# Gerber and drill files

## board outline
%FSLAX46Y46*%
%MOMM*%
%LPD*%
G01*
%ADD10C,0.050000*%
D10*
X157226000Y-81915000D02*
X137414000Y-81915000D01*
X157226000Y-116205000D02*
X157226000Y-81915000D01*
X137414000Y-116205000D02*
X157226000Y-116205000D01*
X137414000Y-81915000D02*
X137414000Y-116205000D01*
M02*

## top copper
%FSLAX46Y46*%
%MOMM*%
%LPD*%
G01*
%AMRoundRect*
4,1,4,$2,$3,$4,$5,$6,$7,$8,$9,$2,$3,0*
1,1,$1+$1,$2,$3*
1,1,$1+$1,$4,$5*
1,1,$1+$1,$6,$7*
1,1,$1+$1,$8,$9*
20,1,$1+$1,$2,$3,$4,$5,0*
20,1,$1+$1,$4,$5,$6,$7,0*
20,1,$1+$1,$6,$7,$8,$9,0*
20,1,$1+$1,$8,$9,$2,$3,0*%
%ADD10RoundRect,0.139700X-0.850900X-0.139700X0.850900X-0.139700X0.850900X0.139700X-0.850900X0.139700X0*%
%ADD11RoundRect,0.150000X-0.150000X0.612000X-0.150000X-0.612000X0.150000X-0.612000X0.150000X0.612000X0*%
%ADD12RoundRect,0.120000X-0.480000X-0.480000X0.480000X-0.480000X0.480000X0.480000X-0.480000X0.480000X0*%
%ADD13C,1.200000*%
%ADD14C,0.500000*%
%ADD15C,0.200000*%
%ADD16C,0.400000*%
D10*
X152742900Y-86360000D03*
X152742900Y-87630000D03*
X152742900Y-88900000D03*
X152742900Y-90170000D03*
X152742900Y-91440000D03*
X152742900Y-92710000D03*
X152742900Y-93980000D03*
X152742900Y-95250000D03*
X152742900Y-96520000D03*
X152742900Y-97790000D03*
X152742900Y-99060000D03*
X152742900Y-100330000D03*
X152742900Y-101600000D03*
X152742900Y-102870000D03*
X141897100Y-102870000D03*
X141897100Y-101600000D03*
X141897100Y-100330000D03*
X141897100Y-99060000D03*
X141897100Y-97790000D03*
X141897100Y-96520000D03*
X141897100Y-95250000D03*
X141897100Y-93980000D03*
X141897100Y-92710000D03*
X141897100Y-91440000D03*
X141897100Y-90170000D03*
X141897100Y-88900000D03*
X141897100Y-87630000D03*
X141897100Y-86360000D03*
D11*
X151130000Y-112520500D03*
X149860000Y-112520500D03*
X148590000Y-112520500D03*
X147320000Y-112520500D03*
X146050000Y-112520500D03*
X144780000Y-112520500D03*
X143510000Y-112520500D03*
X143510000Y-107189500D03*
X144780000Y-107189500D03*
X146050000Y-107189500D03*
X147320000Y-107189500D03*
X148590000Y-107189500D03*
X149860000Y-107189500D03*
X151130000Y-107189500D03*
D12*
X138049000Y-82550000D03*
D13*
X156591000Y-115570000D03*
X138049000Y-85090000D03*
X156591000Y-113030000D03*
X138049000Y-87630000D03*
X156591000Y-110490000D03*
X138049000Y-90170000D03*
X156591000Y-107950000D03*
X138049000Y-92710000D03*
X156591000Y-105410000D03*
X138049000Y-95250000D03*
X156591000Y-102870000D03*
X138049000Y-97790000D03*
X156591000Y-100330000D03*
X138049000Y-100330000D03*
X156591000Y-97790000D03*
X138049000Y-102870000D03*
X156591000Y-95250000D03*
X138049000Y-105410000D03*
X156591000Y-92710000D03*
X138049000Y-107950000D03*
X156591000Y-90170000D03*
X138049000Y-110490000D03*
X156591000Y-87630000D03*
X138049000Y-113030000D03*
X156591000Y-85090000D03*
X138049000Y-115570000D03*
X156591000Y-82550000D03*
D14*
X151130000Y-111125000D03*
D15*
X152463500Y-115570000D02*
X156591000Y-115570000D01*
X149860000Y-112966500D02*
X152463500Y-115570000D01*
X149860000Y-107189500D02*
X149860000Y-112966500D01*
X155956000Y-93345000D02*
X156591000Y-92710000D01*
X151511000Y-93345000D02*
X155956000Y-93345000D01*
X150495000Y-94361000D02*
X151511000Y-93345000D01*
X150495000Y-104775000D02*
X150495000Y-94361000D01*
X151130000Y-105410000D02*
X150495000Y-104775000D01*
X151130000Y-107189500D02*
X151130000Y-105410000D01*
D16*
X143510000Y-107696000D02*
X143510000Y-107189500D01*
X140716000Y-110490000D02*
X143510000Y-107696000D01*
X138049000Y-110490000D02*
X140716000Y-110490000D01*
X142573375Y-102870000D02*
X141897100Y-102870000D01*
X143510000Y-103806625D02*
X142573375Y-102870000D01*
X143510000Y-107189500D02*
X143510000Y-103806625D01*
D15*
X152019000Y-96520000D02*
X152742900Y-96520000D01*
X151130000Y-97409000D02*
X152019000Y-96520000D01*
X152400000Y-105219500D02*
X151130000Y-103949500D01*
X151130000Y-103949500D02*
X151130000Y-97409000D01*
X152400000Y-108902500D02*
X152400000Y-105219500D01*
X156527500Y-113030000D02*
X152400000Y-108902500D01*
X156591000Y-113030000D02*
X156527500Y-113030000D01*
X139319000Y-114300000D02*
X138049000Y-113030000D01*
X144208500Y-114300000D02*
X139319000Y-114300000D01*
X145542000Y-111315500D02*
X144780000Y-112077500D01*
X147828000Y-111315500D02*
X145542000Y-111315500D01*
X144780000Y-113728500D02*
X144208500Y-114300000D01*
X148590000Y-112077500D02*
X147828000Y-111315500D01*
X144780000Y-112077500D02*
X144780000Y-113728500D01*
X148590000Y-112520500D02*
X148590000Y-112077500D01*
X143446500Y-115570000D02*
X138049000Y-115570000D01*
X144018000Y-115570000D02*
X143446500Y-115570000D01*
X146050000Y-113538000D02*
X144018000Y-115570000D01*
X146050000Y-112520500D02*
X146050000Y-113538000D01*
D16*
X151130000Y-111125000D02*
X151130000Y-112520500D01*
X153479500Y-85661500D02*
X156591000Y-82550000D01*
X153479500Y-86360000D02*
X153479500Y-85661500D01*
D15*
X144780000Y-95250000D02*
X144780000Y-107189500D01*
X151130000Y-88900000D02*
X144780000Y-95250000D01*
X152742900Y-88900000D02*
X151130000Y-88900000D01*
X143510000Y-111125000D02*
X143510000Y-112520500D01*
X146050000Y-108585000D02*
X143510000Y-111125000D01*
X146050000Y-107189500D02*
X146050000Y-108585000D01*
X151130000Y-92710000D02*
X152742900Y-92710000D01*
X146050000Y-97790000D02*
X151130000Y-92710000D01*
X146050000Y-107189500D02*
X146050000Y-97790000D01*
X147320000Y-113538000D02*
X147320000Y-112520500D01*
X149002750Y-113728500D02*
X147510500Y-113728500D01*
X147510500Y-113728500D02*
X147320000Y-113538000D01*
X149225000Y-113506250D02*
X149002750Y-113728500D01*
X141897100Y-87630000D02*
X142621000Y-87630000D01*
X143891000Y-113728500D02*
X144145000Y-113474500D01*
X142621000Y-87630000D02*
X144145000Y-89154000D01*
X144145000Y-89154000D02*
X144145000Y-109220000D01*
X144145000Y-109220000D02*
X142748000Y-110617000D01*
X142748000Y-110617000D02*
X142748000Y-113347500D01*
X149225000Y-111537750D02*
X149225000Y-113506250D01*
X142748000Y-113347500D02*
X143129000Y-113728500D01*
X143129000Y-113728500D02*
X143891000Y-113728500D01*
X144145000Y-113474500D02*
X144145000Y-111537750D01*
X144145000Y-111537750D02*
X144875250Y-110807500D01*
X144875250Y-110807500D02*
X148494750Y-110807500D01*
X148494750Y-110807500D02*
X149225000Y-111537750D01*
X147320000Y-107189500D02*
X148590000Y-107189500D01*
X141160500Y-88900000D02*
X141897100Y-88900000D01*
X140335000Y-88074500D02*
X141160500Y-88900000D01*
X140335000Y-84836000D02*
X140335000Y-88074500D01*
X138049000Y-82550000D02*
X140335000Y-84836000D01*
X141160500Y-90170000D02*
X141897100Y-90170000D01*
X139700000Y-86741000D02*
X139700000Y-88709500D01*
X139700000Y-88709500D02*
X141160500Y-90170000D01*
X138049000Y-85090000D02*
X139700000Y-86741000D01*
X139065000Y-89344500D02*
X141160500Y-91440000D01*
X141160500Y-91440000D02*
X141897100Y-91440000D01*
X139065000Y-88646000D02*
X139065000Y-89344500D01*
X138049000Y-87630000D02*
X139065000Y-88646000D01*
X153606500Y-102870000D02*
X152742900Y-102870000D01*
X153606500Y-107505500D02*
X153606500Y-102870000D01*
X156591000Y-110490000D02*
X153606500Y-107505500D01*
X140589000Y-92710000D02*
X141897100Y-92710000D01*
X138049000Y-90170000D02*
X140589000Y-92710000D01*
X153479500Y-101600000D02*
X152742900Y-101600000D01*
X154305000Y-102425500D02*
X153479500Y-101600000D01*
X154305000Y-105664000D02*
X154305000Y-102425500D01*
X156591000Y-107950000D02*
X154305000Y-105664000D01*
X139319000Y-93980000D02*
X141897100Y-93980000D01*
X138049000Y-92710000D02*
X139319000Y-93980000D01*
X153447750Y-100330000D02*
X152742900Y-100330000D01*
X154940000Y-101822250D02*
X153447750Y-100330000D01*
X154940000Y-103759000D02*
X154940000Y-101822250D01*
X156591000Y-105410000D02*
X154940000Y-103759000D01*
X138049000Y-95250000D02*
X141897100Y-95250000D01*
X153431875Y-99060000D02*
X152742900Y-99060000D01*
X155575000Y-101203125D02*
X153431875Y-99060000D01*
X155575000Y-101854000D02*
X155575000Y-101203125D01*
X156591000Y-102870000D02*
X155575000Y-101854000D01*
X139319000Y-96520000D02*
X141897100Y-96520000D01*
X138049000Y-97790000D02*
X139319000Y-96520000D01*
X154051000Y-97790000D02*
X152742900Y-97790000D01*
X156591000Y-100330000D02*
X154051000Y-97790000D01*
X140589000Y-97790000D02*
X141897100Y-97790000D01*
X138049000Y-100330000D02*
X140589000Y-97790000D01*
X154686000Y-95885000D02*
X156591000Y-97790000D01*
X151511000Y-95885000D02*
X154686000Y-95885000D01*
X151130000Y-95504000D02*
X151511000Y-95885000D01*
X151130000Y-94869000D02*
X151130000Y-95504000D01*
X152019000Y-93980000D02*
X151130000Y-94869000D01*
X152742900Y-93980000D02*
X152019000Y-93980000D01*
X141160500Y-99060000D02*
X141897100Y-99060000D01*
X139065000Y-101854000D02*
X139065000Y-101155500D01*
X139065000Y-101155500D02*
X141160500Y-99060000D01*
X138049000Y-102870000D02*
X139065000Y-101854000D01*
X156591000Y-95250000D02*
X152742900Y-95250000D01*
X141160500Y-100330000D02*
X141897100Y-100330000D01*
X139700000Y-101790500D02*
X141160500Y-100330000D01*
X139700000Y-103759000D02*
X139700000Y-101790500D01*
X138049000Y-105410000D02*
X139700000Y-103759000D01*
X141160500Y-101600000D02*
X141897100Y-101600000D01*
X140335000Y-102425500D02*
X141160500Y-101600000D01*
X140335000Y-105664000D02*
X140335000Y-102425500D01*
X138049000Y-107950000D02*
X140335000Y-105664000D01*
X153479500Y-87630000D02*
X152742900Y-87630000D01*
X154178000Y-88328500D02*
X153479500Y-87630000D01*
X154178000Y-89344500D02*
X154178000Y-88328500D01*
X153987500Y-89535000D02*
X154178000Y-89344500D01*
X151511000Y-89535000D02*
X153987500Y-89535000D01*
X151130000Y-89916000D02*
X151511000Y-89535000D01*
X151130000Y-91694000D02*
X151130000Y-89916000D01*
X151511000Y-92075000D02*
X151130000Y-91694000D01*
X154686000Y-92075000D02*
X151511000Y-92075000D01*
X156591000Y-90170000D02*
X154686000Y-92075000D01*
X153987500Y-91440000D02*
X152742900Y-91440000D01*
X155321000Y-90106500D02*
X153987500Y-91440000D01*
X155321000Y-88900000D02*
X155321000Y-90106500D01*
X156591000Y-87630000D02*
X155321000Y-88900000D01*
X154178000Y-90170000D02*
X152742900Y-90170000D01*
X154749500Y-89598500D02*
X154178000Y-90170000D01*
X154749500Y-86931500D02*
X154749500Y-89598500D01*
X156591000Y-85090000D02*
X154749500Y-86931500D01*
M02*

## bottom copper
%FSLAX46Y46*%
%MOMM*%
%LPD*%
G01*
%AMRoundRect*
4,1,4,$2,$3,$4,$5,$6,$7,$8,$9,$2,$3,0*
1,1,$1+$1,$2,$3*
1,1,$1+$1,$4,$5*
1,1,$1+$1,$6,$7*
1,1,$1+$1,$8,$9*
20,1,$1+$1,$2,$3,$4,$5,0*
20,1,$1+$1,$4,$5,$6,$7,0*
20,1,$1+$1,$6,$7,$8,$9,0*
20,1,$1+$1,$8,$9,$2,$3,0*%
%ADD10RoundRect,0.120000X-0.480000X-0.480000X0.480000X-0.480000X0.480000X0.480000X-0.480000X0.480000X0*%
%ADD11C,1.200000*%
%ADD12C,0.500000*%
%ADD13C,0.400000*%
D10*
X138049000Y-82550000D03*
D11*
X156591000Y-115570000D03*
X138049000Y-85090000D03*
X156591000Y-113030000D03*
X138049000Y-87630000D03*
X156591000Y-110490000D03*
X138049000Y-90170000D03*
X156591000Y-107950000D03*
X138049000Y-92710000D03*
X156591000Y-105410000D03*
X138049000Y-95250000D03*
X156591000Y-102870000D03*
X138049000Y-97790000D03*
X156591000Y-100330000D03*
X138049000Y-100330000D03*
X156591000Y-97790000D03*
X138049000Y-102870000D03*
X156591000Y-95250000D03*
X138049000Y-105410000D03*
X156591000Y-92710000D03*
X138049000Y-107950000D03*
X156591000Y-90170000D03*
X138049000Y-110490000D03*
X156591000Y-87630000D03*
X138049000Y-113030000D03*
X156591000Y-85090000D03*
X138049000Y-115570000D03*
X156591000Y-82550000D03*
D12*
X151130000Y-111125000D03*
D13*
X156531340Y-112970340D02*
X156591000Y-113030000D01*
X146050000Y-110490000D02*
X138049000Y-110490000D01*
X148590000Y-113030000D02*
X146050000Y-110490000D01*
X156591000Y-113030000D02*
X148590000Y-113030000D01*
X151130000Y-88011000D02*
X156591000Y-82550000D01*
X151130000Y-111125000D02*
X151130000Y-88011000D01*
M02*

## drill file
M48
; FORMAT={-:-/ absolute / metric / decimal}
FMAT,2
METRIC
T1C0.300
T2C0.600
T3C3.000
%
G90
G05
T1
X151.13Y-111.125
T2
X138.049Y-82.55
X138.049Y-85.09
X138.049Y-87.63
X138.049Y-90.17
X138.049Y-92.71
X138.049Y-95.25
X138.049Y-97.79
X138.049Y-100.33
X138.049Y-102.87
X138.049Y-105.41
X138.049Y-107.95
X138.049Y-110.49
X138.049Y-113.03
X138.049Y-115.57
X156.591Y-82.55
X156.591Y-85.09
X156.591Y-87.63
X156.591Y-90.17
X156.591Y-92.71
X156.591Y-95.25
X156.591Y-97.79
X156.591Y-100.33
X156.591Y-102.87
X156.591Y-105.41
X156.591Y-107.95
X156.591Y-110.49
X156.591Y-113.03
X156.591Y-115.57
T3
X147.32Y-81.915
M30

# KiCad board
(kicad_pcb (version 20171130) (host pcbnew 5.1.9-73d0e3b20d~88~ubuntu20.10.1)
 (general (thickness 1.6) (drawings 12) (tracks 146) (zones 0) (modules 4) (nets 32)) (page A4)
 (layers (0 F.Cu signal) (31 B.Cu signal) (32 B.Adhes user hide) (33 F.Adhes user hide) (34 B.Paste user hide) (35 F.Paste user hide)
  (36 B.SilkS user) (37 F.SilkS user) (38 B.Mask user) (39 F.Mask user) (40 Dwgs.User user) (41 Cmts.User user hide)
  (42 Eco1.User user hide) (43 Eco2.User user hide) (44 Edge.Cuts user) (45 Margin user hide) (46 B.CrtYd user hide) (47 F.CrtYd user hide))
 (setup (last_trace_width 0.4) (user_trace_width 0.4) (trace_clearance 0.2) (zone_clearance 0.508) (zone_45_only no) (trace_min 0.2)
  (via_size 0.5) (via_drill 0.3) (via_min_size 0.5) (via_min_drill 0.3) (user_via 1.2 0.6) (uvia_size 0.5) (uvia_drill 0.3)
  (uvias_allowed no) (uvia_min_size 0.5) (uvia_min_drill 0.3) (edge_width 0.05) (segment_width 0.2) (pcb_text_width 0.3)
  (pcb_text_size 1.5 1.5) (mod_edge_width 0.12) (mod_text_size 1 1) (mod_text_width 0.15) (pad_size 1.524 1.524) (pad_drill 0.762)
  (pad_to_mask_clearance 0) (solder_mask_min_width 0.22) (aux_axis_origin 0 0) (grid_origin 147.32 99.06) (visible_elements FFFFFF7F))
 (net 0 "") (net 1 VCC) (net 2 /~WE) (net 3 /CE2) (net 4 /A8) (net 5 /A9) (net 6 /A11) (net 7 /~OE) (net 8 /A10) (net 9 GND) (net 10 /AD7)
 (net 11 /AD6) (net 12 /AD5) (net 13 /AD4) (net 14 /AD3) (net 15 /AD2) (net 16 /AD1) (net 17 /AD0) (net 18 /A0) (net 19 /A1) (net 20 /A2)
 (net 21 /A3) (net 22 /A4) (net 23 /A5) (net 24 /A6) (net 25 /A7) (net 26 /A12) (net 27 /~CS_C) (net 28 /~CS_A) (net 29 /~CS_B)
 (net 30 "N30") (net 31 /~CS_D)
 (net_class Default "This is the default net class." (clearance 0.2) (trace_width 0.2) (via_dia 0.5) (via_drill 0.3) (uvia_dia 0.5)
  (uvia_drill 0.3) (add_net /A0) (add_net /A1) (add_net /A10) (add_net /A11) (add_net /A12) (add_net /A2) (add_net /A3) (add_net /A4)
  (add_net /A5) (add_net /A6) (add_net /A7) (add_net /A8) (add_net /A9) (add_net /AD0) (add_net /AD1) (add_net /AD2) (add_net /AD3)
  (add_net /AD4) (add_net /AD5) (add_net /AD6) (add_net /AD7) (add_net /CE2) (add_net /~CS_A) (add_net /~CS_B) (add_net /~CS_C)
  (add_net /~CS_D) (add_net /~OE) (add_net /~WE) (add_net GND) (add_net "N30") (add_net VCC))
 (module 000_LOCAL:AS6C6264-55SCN (layer F.Cu) (at 147.32 94.615)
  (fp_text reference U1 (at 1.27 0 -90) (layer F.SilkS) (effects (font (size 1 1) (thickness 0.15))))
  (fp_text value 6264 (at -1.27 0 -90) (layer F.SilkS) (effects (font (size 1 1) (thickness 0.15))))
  (pad 28 smd roundrect (at 5.4229 -8.255) (size 1.9812 0.5588) (layers F.Cu F.Paste F.Mask) (roundrect_rratio 0.25) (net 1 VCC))
  (pad 27 smd roundrect (at 5.4229 -6.985) (size 1.9812 0.5588) (layers F.Cu F.Paste F.Mask) (roundrect_rratio 0.25) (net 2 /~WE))
  (pad 26 smd roundrect (at 5.4229 -5.715) (size 1.9812 0.5588) (layers F.Cu F.Paste F.Mask) (roundrect_rratio 0.25) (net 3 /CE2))
  (pad 25 smd roundrect (at 5.4229 -4.445) (size 1.9812 0.5588) (layers F.Cu F.Paste F.Mask) (roundrect_rratio 0.25) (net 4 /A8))
  (pad 24 smd roundrect (at 5.4229 -3.175) (size 1.9812 0.5588) (layers F.Cu F.Paste F.Mask) (roundrect_rratio 0.25) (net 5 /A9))
  (pad 23 smd roundrect (at 5.4229 -1.905) (size 1.9812 0.5588) (layers F.Cu F.Paste F.Mask) (roundrect_rratio 0.25) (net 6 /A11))
  (pad 22 smd roundrect (at 5.4229 -0.635) (size 1.9812 0.5588) (layers F.Cu F.Paste F.Mask) (roundrect_rratio 0.25) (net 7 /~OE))
  (pad 21 smd roundrect (at 5.4229 0.635) (size 1.9812 0.5588) (layers F.Cu F.Paste F.Mask) (roundrect_rratio 0.25) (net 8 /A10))
  (pad 20 smd roundrect (at 5.4229 1.905) (size 1.9812 0.5588) (layers F.Cu F.Paste F.Mask) (roundrect_rratio 0.25) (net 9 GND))
  (pad 19 smd roundrect (at 5.4229 3.175) (size 1.9812 0.5588) (layers F.Cu F.Paste F.Mask) (roundrect_rratio 0.25) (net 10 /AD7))
  (pad 18 smd roundrect (at 5.4229 4.445) (size 1.9812 0.5588) (layers F.Cu F.Paste F.Mask) (roundrect_rratio 0.25) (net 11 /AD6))
  (pad 17 smd roundrect (at 5.4229 5.715) (size 1.9812 0.5588) (layers F.Cu F.Paste F.Mask) (roundrect_rratio 0.25) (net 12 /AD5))
  (pad 16 smd roundrect (at 5.4229 6.985) (size 1.9812 0.5588) (layers F.Cu F.Paste F.Mask) (roundrect_rratio 0.25) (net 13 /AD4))
  (pad 15 smd roundrect (at 5.4229 8.255) (size 1.9812 0.5588) (layers F.Cu F.Paste F.Mask) (roundrect_rratio 0.25) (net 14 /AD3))
  (pad 14 smd roundrect (at -5.4229 8.255) (size 1.9812 0.5588) (layers F.Cu F.Paste F.Mask) (roundrect_rratio 0.25) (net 9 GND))
  (pad 13 smd roundrect (at -5.4229 6.985) (size 1.9812 0.5588) (layers F.Cu F.Paste F.Mask) (roundrect_rratio 0.25) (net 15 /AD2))
  (pad 12 smd roundrect (at -5.4229 5.715) (size 1.9812 0.5588) (layers F.Cu F.Paste F.Mask) (roundrect_rratio 0.25) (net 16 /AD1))
  (pad 11 smd roundrect (at -5.4229 4.445) (size 1.9812 0.5588) (layers F.Cu F.Paste F.Mask) (roundrect_rratio 0.25) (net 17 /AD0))
  (pad 10 smd roundrect (at -5.4229 3.175) (size 1.9812 0.5588) (layers F.Cu F.Paste F.Mask) (roundrect_rratio 0.25) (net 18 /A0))
  (pad 9 smd roundrect (at -5.4229 1.905) (size 1.9812 0.5588) (layers F.Cu F.Paste F.Mask) (roundrect_rratio 0.25) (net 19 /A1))
  (pad 8 smd roundrect (at -5.4229 0.635) (size 1.9812 0.5588) (layers F.Cu F.Paste F.Mask) (roundrect_rratio 0.25) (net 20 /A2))
  (pad 7 smd roundrect (at -5.4229 -0.635) (size 1.9812 0.5588) (layers F.Cu F.Paste F.Mask) (roundrect_rratio 0.25) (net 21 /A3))
  (pad 6 smd roundrect (at -5.4229 -1.905) (size 1.9812 0.5588) (layers F.Cu F.Paste F.Mask) (roundrect_rratio 0.25) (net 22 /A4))
  (pad 5 smd roundrect (at -5.4229 -3.175) (size 1.9812 0.5588) (layers F.Cu F.Paste F.Mask) (roundrect_rratio 0.25) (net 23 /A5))
  (pad 4 smd roundrect (at -5.4229 -4.445) (size 1.9812 0.5588) (layers F.Cu F.Paste F.Mask) (roundrect_rratio 0.25) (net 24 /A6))
  (pad 3 smd roundrect (at -5.4229 -5.715) (size 1.9812 0.5588) (layers F.Cu F.Paste F.Mask) (roundrect_rratio 0.25) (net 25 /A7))
  (pad 2 smd roundrect (at -5.4229 -6.985) (size 1.9812 0.5588) (layers F.Cu F.Paste F.Mask) (roundrect_rratio 0.25) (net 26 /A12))
  (pad 1 smd roundrect (at -5.4229 -8.255) (size 1.9812 0.5588) (layers F.Cu F.Paste F.Mask) (roundrect_rratio 0.25)))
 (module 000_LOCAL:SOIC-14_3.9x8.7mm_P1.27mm (layer F.Cu) (at 147.32 109.855 270) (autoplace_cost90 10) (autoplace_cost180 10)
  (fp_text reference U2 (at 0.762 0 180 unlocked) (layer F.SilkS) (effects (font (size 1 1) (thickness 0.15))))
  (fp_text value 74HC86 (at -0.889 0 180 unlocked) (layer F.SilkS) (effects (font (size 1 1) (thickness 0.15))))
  (pad 14 smd roundrect (at 2.6655 -3.81 270) (size 1.524 0.6) (layers F.Cu F.Paste F.Mask) (roundrect_rratio 0.25) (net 1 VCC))
  (pad 13 smd roundrect (at 2.6655 -2.54 270) (size 1.524 0.6) (layers F.Cu F.Paste F.Mask) (roundrect_rratio 0.25) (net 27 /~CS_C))
  (pad 12 smd roundrect (at 2.6655 -1.27 270) (size 1.524 0.6) (layers F.Cu F.Paste F.Mask) (roundrect_rratio 0.25) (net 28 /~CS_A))
  (pad 11 smd roundrect (at 2.6655 0 270) (size 1.524 0.6) (layers F.Cu F.Paste F.Mask) (roundrect_rratio 0.25) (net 26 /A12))
  (pad 10 smd roundrect (at 2.6655 1.27 270) (size 1.524 0.6) (layers F.Cu F.Paste F.Mask) (roundrect_rratio 0.25) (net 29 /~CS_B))
  (pad 9 smd roundrect (at 2.6655 2.54 270) (size 1.524 0.6) (layers F.Cu F.Paste F.Mask) (roundrect_rratio 0.25) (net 28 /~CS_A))
  (pad 8 smd roundrect (at 2.6655 3.81 270) (size 1.524 0.6) (layers F.Cu F.Paste F.Mask) (roundrect_rratio 0.25) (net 6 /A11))
  (pad 7 smd roundrect (at -2.6655 3.81 270) (size 1.524 0.6) (layers F.Cu F.Paste F.Mask) (roundrect_rratio 0.25) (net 9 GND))
  (pad 6 smd roundrect (at -2.6655 2.54 270) (size 1.524 0.6) (layers F.Cu F.Paste F.Mask) (roundrect_rratio 0.25) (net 3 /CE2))
  (pad 5 smd roundrect (at -2.6655 1.27 270) (size 1.524 0.6) (layers F.Cu F.Paste F.Mask) (roundrect_rratio 0.25) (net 6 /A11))
  (pad 4 smd roundrect (at -2.6655 0 270) (size 1.524 0.6) (layers F.Cu F.Paste F.Mask) (roundrect_rratio 0.25) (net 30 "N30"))
  (pad 3 smd roundrect (at -2.6655 -1.27 270) (size 1.524 0.6) (layers F.Cu F.Paste F.Mask) (roundrect_rratio 0.25) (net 30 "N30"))
  (pad 2 smd roundrect (at -2.6655 -2.54 270) (size 1.524 0.6) (layers F.Cu F.Paste F.Mask) (roundrect_rratio 0.25) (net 27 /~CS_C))
  (pad 1 smd roundrect (at -2.6655 -3.81 270) (size 1.524 0.6) (layers F.Cu F.Paste F.Mask) (roundrect_rratio 0.25) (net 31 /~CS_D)))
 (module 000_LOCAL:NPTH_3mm (layer F.Cu) (at 147.32 81.915)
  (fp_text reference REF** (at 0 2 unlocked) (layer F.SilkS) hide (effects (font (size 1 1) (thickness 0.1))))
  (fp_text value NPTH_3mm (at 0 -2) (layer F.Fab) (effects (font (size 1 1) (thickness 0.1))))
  (pad "" np_thru_hole circle (at 0 0) (size 3 3) (drill 3) (layers *.Cu *.Mask)))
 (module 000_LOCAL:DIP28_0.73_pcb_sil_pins (layer F.Cu) (at 147.32 99.06)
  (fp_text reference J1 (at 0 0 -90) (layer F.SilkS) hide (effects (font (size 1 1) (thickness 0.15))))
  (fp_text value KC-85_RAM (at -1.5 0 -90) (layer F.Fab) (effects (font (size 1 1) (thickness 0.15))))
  (pad 1 thru_hole roundrect (at -9.271 -16.51) (size 1.2 1.2) (drill 0.6) (layers *.Cu *.Mask) (roundrect_rratio 0.1) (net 25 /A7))
  (pad 15 thru_hole circle (at 9.271 16.51) (size 1.2 1.2) (drill 0.6) (layers *.Cu *.Mask) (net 27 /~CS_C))
  (pad 2 thru_hole circle (at -9.271 -13.97) (size 1.2 1.2) (drill 0.6) (layers *.Cu *.Mask) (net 24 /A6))
  (pad 16 thru_hole circle (at 9.271 13.97) (size 1.2 1.2) (drill 0.6) (layers *.Cu *.Mask) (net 9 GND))
  (pad 3 thru_hole circle (at -9.271 -11.43) (size 1.2 1.2) (drill 0.6) (layers *.Cu *.Mask) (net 23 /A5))
  (pad 17 thru_hole circle (at 9.271 11.43) (size 1.2 1.2) (drill 0.6) (layers *.Cu *.Mask) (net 14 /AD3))
  (pad 4 thru_hole circle (at -9.271 -8.89) (size 1.2 1.2) (drill 0.6) (layers *.Cu *.Mask) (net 22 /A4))
  (pad 18 thru_hole circle (at 9.271 8.89) (size 1.2 1.2) (drill 0.6) (layers *.Cu *.Mask) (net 13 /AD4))
  (pad 5 thru_hole circle (at -9.271 -6.35) (size 1.2 1.2) (drill 0.6) (layers *.Cu *.Mask) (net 21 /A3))
  (pad 19 thru_hole circle (at 9.271 6.35) (size 1.2 1.2) (drill 0.6) (layers *.Cu *.Mask) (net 12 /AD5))
  (pad 6 thru_hole circle (at -9.271 -3.81) (size 1.2 1.2) (drill 0.6) (layers *.Cu *.Mask) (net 20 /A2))
  (pad 20 thru_hole circle (at 9.271 3.81) (size 1.2 1.2) (drill 0.6) (layers *.Cu *.Mask) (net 11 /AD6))
  (pad 7 thru_hole circle (at -9.271 -1.27) (size 1.2 1.2) (drill 0.6) (layers *.Cu *.Mask) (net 19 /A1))
  (pad 21 thru_hole circle (at 9.271 1.27) (size 1.2 1.2) (drill 0.6) (layers *.Cu *.Mask) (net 10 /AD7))
  (pad 8 thru_hole circle (at -9.271 1.27) (size 1.2 1.2) (drill 0.6) (layers *.Cu *.Mask) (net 18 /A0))
  (pad 22 thru_hole circle (at 9.271 -1.27) (size 1.2 1.2) (drill 0.6) (layers *.Cu *.Mask) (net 7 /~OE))
  (pad 9 thru_hole circle (at -9.271 3.81) (size 1.2 1.2) (drill 0.6) (layers *.Cu *.Mask) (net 17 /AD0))
  (pad 23 thru_hole circle (at 9.271 -3.81) (size 1.2 1.2) (drill 0.6) (layers *.Cu *.Mask) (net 8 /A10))
  (pad 10 thru_hole circle (at -9.271 6.35) (size 1.2 1.2) (drill 0.6) (layers *.Cu *.Mask) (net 16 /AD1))
  (pad 24 thru_hole circle (at 9.271 -6.35) (size 1.2 1.2) (drill 0.6) (layers *.Cu *.Mask) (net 31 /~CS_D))
  (pad 11 thru_hole circle (at -9.271 8.89) (size 1.2 1.2) (drill 0.6) (layers *.Cu *.Mask) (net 15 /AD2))
  (pad 25 thru_hole circle (at 9.271 -8.89) (size 1.2 1.2) (drill 0.6) (layers *.Cu *.Mask) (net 2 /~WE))
  (pad 12 thru_hole circle (at -9.271 11.43) (size 1.2 1.2) (drill 0.6) (layers *.Cu *.Mask) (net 9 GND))
  (pad 26 thru_hole circle (at 9.271 -11.43) (size 1.2 1.2) (drill 0.6) (layers *.Cu *.Mask) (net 5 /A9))
  (pad 13 thru_hole circle (at -9.271 13.97) (size 1.2 1.2) (drill 0.6) (layers *.Cu *.Mask) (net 28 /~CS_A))
  (pad 27 thru_hole circle (at 9.271 -13.97) (size 1.2 1.2) (drill 0.6) (layers *.Cu *.Mask) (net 4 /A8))
  (pad 14 thru_hole circle (at -9.271 16.51) (size 1.2 1.2) (drill 0.6) (layers *.Cu *.Mask) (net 29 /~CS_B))
  (pad 28 thru_hole circle (at 9.271 -16.51) (size 1.2 1.2) (drill 0.6) (layers *.Cu *.Mask) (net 1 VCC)))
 (gr_line (start 157.226 81.915) (end 137.414 81.915) (layer Edge.Cuts) (width 0.05))
 (gr_line (start 157.226 116.205) (end 157.226 81.915) (layer Edge.Cuts) (width 0.05))
 (gr_line (start 137.414 116.205) (end 157.226 116.205) (layer Edge.Cuts) (width 0.05))
 (gr_line (start 137.414 81.915) (end 137.414 116.205) (layer Edge.Cuts) (width 0.05))
 (segment (start 152.4635 115.57) (end 156.591 115.57) (width 0.2) (layer F.Cu) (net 27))
 (segment (start 149.86 112.9665) (end 152.4635 115.57) (width 0.2) (layer F.Cu) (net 27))
 (segment (start 149.86 107.1895) (end 149.86 112.9665) (width 0.2) (layer F.Cu) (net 27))
 (segment (start 155.956 93.345) (end 156.591 92.71) (width 0.2) (layer F.Cu) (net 31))
 (segment (start 151.511 93.345) (end 155.956 93.345) (width 0.2) (layer F.Cu) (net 31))
 (segment (start 150.495 94.361) (end 151.511 93.345) (width 0.2) (layer F.Cu) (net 31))
 (segment (start 150.495 104.775) (end 150.495 94.361) (width 0.2) (layer F.Cu) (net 31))
 (segment (start 151.13 105.41) (end 150.495 104.775) (width 0.2) (layer F.Cu) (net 31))
 (segment (start 151.13 107.1895) (end 151.13 105.41) (width 0.2) (layer F.Cu) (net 31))
 (segment (start 156.53134 112.97034) (end 156.591 113.03) (width 0.4) (layer B.Cu) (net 9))
 (segment (start 143.51 107.696) (end 143.51 107.1895) (width 0.4) (layer F.Cu) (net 9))
 (segment (start 140.716 110.49) (end 143.51 107.696) (width 0.4) (layer F.Cu) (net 9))
 (segment (start 138.049 110.49) (end 140.716 110.49) (width 0.4) (layer F.Cu) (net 9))
 (segment (start 142.573375 102.87) (end 141.8971 102.87) (width 0.4) (layer F.Cu) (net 9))
 (segment (start 143.51 103.806625) (end 142.573375 102.87) (width 0.4) (layer F.Cu) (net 9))
 (segment (start 143.51 107.1895) (end 143.51 103.806625) (width 0.4) (layer F.Cu) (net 9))
 (segment (start 146.05 110.49) (end 138.049 110.49) (width 0.4) (layer B.Cu) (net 9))
 (segment (start 148.59 113.03) (end 146.05 110.49) (width 0.4) (layer B.Cu) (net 9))
 (segment (start 156.591 113.03) (end 148.59 113.03) (width 0.4) (layer B.Cu) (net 9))
 (segment (start 152.019 96.52) (end 152.7429 96.52) (width 0.2) (layer F.Cu) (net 9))
 (segment (start 151.13 97.409) (end 152.019 96.52) (width 0.2) (layer F.Cu) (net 9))
 (segment (start 152.4 105.2195) (end 151.13 103.9495) (width 0.2) (layer F.Cu) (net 9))
 (segment (start 151.13 103.9495) (end 151.13 97.409) (width 0.2) (layer F.Cu) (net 9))
 (segment (start 152.4 108.9025) (end 152.4 105.2195) (width 0.2) (layer F.Cu) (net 9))
 (segment (start 156.5275 113.03) (end 152.4 108.9025) (width 0.2) (layer F.Cu) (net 9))
 (segment (start 156.591 113.03) (end 156.5275 113.03) (width 0.2) (layer F.Cu) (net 9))
 (segment (start 139.319 114.3) (end 138.049 113.03) (width 0.2) (layer F.Cu) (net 28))
 (segment (start 144.2085 114.3) (end 139.319 114.3) (width 0.2) (layer F.Cu) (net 28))
 (segment (start 145.542 111.3155) (end 144.78 112.0775) (width 0.2) (layer F.Cu) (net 28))
 (segment (start 147.828 111.3155) (end 145.542 111.3155) (width 0.2) (layer F.Cu) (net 28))
 (segment (start 144.78 113.7285) (end 144.2085 114.3) (width 0.2) (layer F.Cu) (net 28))
 (segment (start 148.59 112.0775) (end 147.828 111.3155) (width 0.2) (layer F.Cu) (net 28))
 (segment (start 144.78 112.0775) (end 144.78 113.7285) (width 0.2) (layer F.Cu) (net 28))
 (segment (start 148.59 112.5205) (end 148.59 112.0775) (width 0.2) (layer F.Cu) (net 28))
 (segment (start 143.4465 115.57) (end 138.049 115.57) (width 0.2) (layer F.Cu) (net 29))
 (segment (start 144.018 115.57) (end 143.4465 115.57) (width 0.2) (layer F.Cu) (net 29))
 (segment (start 146.05 113.538) (end 144.018 115.57) (width 0.2) (layer F.Cu) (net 29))
 (segment (start 146.05 112.5205) (end 146.05 113.538) (width 0.2) (layer F.Cu) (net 29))
 (via (at 151.13 111.125) (size 0.5) (drill 0.3) (layers F.Cu B.Cu) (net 1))
 (segment (start 151.13 111.125) (end 151.13 112.5205) (width 0.4) (layer F.Cu) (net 1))
 (segment (start 151.13 88.011) (end 156.591 82.55) (width 0.4) (layer B.Cu) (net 1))
 (segment (start 151.13 111.125) (end 151.13 88.011) (width 0.4) (layer B.Cu) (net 1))
 (segment (start 153.4795 85.6615) (end 156.591 82.55) (width 0.4) (layer F.Cu) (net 1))
 (segment (start 153.4795 86.36) (end 153.4795 85.6615) (width 0.4) (layer F.Cu) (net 1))
 (segment (start 144.78 95.25) (end 144.78 107.1895) (width 0.2) (layer F.Cu) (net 3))
 (segment (start 151.13 88.9) (end 144.78 95.25) (width 0.2) (layer F.Cu) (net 3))
 (segment (start 152.7429 88.9) (end 151.13 88.9) (width 0.2) (layer F.Cu) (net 3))
 (segment (start 143.51 111.125) (end 143.51 112.5205) (width 0.2) (layer F.Cu) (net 6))
 (segment (start 146.05 108.585) (end 143.51 111.125) (width 0.2) (layer F.Cu) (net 6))
 (segment (start 146.05 107.1895) (end 146.05 108.585) (width 0.2) (layer F.Cu) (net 6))
 (segment (start 151.13 92.71) (end 152.7429 92.71) (width 0.2) (layer F.Cu) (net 6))
 (segment (start 146.05 97.79) (end 151.13 92.71) (width 0.2) (layer F.Cu) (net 6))
 (segment (start 146.05 107.1895) (end 146.05 97.79) (width 0.2) (layer F.Cu) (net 6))
 (segment (start 147.32 113.538) (end 147.32 112.5205) (width 0.2) (layer F.Cu) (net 26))
 (segment (start 149.00275 113.7285) (end 147.5105 113.7285) (width 0.2) (layer F.Cu) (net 26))
 (segment (start 147.5105 113.7285) (end 147.32 113.538) (width 0.2) (layer F.Cu) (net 26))
 (segment (start 149.225 113.50625) (end 149.00275 113.7285) (width 0.2) (layer F.Cu) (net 26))
 (segment (start 141.8971 87.63) (end 142.621 87.63) (width 0.2) (layer F.Cu) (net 26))
 (segment (start 143.891 113.7285) (end 144.145 113.4745) (width 0.2) (layer F.Cu) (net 26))
 (segment (start 142.621 87.63) (end 144.145 89.154) (width 0.2) (layer F.Cu) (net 26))
 (segment (start 144.145 89.154) (end 144.145 109.22) (width 0.2) (layer F.Cu) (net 26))
 (segment (start 144.145 109.22) (end 142.748 110.617) (width 0.2) (layer F.Cu) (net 26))
 (segment (start 142.748 110.617) (end 142.748 113.3475) (width 0.2) (layer F.Cu) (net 26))
 (segment (start 149.225 111.53775) (end 149.225 113.50625) (width 0.2) (layer F.Cu) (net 26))
 (segment (start 142.748 113.3475) (end 143.129 113.7285) (width 0.2) (layer F.Cu) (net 26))
 (segment (start 143.129 113.7285) (end 143.891 113.7285) (width 0.2) (layer F.Cu) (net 26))
 (segment (start 144.145 113.4745) (end 144.145 111.53775) (width 0.2) (layer F.Cu) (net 26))
 (segment (start 144.145 111.53775) (end 144.87525 110.8075) (width 0.2) (layer F.Cu) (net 26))
 (segment (start 144.87525 110.8075) (end 148.49475 110.8075) (width 0.2) (layer F.Cu) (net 26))
 (segment (start 148.49475 110.8075) (end 149.225 111.53775) (width 0.2) (layer F.Cu) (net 26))
 (segment (start 147.32 107.1895) (end 148.59 107.1895) (width 0.2) (layer F.Cu) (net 30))
 (segment (start 141.1605 88.9) (end 141.8971 88.9) (width 0.2) (layer F.Cu) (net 25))
 (segment (start 140.335 88.0745) (end 141.1605 88.9) (width 0.2) (layer F.Cu) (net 25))
 (segment (start 140.335 84.836) (end 140.335 88.0745) (width 0.2) (layer F.Cu) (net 25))
 (segment (start 138.049 82.55) (end 140.335 84.836) (width 0.2) (layer F.Cu) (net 25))
 (segment (start 141.1605 90.17) (end 141.8971 90.17) (width 0.2) (layer F.Cu) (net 24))
 (segment (start 139.7 86.741) (end 139.7 88.7095) (width 0.2) (layer F.Cu) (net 24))
 (segment (start 139.7 88.7095) (end 141.1605 90.17) (width 0.2) (layer F.Cu) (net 24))
 (segment (start 138.049 85.09) (end 139.7 86.741) (width 0.2) (layer F.Cu) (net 24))
 (segment (start 139.065 89.3445) (end 141.1605 91.44) (width 0.2) (layer F.Cu) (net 23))
 (segment (start 141.1605 91.44) (end 141.8971 91.44) (width 0.2) (layer F.Cu) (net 23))
 (segment (start 139.065 88.646) (end 139.065 89.3445) (width 0.2) (layer F.Cu) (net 23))
 (segment (start 138.049 87.63) (end 139.065 88.646) (width 0.2) (layer F.Cu) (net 23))
 (segment (start 153.6065 102.87) (end 152.7429 102.87) (width 0.2) (layer F.Cu) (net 14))
 (segment (start 153.6065 107.5055) (end 153.6065 102.87) (width 0.2) (layer F.Cu) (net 14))
 (segment (start 156.591 110.49) (end 153.6065 107.5055) (width 0.2) (layer F.Cu) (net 14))
 (segment (start 140.589 92.71) (end 141.8971 92.71) (width 0.2) (layer F.Cu) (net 22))
 (segment (start 138.049 90.17) (end 140.589 92.71) (width 0.2) (layer F.Cu) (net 22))
 (segment (start 153.4795 101.6) (end 152.7429 101.6) (width 0.2) (layer F.Cu) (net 13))
 (segment (start 154.305 102.4255) (end 153.4795 101.6) (width 0.2) (layer F.Cu) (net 13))
 (segment (start 154.305 105.664) (end 154.305 102.4255) (width 0.2) (layer F.Cu) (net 13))
 (segment (start 156.591 107.95) (end 154.305 105.664) (width 0.2) (layer F.Cu) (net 13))
 (segment (start 139.319 93.98) (end 141.8971 93.98) (width 0.2) (layer F.Cu) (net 21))
 (segment (start 138.049 92.71) (end 139.319 93.98) (width 0.2) (layer F.Cu) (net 21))
 (segment (start 153.44775 100.33) (end 152.7429 100.33) (width 0.2) (layer F.Cu) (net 12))
 (segment (start 154.94 101.82225) (end 153.44775 100.33) (width 0.2) (layer F.Cu) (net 12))
 (segment (start 154.94 103.759) (end 154.94 101.82225) (width 0.2) (layer F.Cu) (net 12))
 (segment (start 156.591 105.41) (end 154.94 103.759) (width 0.2) (layer F.Cu) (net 12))
 (segment (start 138.049 95.25) (end 141.8971 95.25) (width 0.2) (layer F.Cu) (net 20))
 (segment (start 153.431875 99.06) (end 152.7429 99.06) (width 0.2) (layer F.Cu) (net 11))
 (segment (start 155.575 101.203125) (end 153.431875 99.06) (width 0.2) (layer F.Cu) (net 11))
 (segment (start 155.575 101.854) (end 155.575 101.203125) (width 0.2) (layer F.Cu) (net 11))
 (segment (start 156.591 102.87) (end 155.575 101.854) (width 0.2) (layer F.Cu) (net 11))
 (segment (start 139.319 96.52) (end 141.8971 96.52) (width 0.2) (layer F.Cu) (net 19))
 (segment (start 138.049 97.79) (end 139.319 96.52) (width 0.2) (layer F.Cu) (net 19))
 (segment (start 154.051 97.79) (end 152.7429 97.79) (width 0.2) (layer F.Cu) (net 10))
 (segment (start 156.591 100.33) (end 154.051 97.79) (width 0.2) (layer F.Cu) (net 10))
 (segment (start 140.589 97.79) (end 141.8971 97.79) (width 0.2) (layer F.Cu) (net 18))
 (segment (start 138.049 100.33) (end 140.589 97.79) (width 0.2) (layer F.Cu) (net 18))
 (segment (start 154.686 95.885) (end 156.591 97.79) (width 0.2) (layer F.Cu) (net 7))
 (segment (start 151.511 95.885) (end 154.686 95.885) (width 0.2) (layer F.Cu) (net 7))
 (segment (start 151.13 95.504) (end 151.511 95.885) (width 0.2) (layer F.Cu) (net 7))
 (segment (start 151.13 94.869) (end 151.13 95.504) (width 0.2) (layer F.Cu) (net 7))
 (segment (start 152.019 93.98) (end 151.13 94.869) (width 0.2) (layer F.Cu) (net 7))
 (segment (start 152.7429 93.98) (end 152.019 93.98) (width 0.2) (layer F.Cu) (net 7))
 (segment (start 141.1605 99.06) (end 141.8971 99.06) (width 0.2) (layer F.Cu) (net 17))
 (segment (start 139.065 101.854) (end 139.065 101.1555) (width 0.2) (layer F.Cu) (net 17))
 (segment (start 139.065 101.1555) (end 141.1605 99.06) (width 0.2) (layer F.Cu) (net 17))
 (segment (start 138.049 102.87) (end 139.065 101.854) (width 0.2) (layer F.Cu) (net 17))
 (segment (start 156.591 95.25) (end 152.7429 95.25) (width 0.2) (layer F.Cu) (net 8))
 (segment (start 141.1605 100.33) (end 141.8971 100.33) (width 0.2) (layer F.Cu) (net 16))
 (segment (start 139.7 101.7905) (end 141.1605 100.33) (width 0.2) (layer F.Cu) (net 16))
 (segment (start 139.7 103.759) (end 139.7 101.7905) (width 0.2) (layer F.Cu) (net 16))
 (segment (start 138.049 105.41) (end 139.7 103.759) (width 0.2) (layer F.Cu) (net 16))
 (segment (start 141.1605 101.6) (end 141.8971 101.6) (width 0.2) (layer F.Cu) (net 15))
 (segment (start 140.335 102.4255) (end 141.1605 101.6) (width 0.2) (layer F.Cu) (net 15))
 (segment (start 140.335 105.664) (end 140.335 102.4255) (width 0.2) (layer F.Cu) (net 15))
 (segment (start 138.049 107.95) (end 140.335 105.664) (width 0.2) (layer F.Cu) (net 15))
 (segment (start 153.4795 87.63) (end 152.7429 87.63) (width 0.2) (layer F.Cu) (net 2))
 (segment (start 154.178 88.3285) (end 153.4795 87.63) (width 0.2) (layer F.Cu) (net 2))
 (segment (start 154.178 89.3445) (end 154.178 88.3285) (width 0.2) (layer F.Cu) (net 2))
 (segment (start 153.9875 89.535) (end 154.178 89.3445) (width 0.2) (layer F.Cu) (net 2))
 (segment (start 151.511 89.535) (end 153.9875 89.535) (width 0.2) (layer F.Cu) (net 2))
 (segment (start 151.13 89.916) (end 151.511 89.535) (width 0.2) (layer F.Cu) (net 2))
 (segment (start 151.13 91.694) (end 151.13 89.916) (width 0.2) (layer F.Cu) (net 2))
 (segment (start 151.511 92.075) (end 151.13 91.694) (width 0.2) (layer F.Cu) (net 2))
 (segment (start 154.686 92.075) (end 151.511 92.075) (width 0.2) (layer F.Cu) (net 2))
 (segment (start 156.591 90.17) (end 154.686 92.075) (width 0.2) (layer F.Cu) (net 2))
 (segment (start 153.9875 91.44) (end 152.7429 91.44) (width 0.2) (layer F.Cu) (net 5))
 (segment (start 155.321 90.1065) (end 153.9875 91.44) (width 0.2) (layer F.Cu) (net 5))
 (segment (start 155.321 88.9) (end 155.321 90.1065) (width 0.2) (layer F.Cu) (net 5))
 (segment (start 156.591 87.63) (end 155.321 88.9) (width 0.2) (layer F.Cu) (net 5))
 (segment (start 154.178 90.17) (end 152.7429 90.17) (width 0.2) (layer F.Cu) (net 4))
 (segment (start 154.7495 89.5985) (end 154.178 90.17) (width 0.2) (layer F.Cu) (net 4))
 (segment (start 154.7495 86.9315) (end 154.7495 89.5985) (width 0.2) (layer F.Cu) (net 4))
 (segment (start 156.591 85.09) (end 154.7495 86.9315) (width 0.2) (layer F.Cu) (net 4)))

